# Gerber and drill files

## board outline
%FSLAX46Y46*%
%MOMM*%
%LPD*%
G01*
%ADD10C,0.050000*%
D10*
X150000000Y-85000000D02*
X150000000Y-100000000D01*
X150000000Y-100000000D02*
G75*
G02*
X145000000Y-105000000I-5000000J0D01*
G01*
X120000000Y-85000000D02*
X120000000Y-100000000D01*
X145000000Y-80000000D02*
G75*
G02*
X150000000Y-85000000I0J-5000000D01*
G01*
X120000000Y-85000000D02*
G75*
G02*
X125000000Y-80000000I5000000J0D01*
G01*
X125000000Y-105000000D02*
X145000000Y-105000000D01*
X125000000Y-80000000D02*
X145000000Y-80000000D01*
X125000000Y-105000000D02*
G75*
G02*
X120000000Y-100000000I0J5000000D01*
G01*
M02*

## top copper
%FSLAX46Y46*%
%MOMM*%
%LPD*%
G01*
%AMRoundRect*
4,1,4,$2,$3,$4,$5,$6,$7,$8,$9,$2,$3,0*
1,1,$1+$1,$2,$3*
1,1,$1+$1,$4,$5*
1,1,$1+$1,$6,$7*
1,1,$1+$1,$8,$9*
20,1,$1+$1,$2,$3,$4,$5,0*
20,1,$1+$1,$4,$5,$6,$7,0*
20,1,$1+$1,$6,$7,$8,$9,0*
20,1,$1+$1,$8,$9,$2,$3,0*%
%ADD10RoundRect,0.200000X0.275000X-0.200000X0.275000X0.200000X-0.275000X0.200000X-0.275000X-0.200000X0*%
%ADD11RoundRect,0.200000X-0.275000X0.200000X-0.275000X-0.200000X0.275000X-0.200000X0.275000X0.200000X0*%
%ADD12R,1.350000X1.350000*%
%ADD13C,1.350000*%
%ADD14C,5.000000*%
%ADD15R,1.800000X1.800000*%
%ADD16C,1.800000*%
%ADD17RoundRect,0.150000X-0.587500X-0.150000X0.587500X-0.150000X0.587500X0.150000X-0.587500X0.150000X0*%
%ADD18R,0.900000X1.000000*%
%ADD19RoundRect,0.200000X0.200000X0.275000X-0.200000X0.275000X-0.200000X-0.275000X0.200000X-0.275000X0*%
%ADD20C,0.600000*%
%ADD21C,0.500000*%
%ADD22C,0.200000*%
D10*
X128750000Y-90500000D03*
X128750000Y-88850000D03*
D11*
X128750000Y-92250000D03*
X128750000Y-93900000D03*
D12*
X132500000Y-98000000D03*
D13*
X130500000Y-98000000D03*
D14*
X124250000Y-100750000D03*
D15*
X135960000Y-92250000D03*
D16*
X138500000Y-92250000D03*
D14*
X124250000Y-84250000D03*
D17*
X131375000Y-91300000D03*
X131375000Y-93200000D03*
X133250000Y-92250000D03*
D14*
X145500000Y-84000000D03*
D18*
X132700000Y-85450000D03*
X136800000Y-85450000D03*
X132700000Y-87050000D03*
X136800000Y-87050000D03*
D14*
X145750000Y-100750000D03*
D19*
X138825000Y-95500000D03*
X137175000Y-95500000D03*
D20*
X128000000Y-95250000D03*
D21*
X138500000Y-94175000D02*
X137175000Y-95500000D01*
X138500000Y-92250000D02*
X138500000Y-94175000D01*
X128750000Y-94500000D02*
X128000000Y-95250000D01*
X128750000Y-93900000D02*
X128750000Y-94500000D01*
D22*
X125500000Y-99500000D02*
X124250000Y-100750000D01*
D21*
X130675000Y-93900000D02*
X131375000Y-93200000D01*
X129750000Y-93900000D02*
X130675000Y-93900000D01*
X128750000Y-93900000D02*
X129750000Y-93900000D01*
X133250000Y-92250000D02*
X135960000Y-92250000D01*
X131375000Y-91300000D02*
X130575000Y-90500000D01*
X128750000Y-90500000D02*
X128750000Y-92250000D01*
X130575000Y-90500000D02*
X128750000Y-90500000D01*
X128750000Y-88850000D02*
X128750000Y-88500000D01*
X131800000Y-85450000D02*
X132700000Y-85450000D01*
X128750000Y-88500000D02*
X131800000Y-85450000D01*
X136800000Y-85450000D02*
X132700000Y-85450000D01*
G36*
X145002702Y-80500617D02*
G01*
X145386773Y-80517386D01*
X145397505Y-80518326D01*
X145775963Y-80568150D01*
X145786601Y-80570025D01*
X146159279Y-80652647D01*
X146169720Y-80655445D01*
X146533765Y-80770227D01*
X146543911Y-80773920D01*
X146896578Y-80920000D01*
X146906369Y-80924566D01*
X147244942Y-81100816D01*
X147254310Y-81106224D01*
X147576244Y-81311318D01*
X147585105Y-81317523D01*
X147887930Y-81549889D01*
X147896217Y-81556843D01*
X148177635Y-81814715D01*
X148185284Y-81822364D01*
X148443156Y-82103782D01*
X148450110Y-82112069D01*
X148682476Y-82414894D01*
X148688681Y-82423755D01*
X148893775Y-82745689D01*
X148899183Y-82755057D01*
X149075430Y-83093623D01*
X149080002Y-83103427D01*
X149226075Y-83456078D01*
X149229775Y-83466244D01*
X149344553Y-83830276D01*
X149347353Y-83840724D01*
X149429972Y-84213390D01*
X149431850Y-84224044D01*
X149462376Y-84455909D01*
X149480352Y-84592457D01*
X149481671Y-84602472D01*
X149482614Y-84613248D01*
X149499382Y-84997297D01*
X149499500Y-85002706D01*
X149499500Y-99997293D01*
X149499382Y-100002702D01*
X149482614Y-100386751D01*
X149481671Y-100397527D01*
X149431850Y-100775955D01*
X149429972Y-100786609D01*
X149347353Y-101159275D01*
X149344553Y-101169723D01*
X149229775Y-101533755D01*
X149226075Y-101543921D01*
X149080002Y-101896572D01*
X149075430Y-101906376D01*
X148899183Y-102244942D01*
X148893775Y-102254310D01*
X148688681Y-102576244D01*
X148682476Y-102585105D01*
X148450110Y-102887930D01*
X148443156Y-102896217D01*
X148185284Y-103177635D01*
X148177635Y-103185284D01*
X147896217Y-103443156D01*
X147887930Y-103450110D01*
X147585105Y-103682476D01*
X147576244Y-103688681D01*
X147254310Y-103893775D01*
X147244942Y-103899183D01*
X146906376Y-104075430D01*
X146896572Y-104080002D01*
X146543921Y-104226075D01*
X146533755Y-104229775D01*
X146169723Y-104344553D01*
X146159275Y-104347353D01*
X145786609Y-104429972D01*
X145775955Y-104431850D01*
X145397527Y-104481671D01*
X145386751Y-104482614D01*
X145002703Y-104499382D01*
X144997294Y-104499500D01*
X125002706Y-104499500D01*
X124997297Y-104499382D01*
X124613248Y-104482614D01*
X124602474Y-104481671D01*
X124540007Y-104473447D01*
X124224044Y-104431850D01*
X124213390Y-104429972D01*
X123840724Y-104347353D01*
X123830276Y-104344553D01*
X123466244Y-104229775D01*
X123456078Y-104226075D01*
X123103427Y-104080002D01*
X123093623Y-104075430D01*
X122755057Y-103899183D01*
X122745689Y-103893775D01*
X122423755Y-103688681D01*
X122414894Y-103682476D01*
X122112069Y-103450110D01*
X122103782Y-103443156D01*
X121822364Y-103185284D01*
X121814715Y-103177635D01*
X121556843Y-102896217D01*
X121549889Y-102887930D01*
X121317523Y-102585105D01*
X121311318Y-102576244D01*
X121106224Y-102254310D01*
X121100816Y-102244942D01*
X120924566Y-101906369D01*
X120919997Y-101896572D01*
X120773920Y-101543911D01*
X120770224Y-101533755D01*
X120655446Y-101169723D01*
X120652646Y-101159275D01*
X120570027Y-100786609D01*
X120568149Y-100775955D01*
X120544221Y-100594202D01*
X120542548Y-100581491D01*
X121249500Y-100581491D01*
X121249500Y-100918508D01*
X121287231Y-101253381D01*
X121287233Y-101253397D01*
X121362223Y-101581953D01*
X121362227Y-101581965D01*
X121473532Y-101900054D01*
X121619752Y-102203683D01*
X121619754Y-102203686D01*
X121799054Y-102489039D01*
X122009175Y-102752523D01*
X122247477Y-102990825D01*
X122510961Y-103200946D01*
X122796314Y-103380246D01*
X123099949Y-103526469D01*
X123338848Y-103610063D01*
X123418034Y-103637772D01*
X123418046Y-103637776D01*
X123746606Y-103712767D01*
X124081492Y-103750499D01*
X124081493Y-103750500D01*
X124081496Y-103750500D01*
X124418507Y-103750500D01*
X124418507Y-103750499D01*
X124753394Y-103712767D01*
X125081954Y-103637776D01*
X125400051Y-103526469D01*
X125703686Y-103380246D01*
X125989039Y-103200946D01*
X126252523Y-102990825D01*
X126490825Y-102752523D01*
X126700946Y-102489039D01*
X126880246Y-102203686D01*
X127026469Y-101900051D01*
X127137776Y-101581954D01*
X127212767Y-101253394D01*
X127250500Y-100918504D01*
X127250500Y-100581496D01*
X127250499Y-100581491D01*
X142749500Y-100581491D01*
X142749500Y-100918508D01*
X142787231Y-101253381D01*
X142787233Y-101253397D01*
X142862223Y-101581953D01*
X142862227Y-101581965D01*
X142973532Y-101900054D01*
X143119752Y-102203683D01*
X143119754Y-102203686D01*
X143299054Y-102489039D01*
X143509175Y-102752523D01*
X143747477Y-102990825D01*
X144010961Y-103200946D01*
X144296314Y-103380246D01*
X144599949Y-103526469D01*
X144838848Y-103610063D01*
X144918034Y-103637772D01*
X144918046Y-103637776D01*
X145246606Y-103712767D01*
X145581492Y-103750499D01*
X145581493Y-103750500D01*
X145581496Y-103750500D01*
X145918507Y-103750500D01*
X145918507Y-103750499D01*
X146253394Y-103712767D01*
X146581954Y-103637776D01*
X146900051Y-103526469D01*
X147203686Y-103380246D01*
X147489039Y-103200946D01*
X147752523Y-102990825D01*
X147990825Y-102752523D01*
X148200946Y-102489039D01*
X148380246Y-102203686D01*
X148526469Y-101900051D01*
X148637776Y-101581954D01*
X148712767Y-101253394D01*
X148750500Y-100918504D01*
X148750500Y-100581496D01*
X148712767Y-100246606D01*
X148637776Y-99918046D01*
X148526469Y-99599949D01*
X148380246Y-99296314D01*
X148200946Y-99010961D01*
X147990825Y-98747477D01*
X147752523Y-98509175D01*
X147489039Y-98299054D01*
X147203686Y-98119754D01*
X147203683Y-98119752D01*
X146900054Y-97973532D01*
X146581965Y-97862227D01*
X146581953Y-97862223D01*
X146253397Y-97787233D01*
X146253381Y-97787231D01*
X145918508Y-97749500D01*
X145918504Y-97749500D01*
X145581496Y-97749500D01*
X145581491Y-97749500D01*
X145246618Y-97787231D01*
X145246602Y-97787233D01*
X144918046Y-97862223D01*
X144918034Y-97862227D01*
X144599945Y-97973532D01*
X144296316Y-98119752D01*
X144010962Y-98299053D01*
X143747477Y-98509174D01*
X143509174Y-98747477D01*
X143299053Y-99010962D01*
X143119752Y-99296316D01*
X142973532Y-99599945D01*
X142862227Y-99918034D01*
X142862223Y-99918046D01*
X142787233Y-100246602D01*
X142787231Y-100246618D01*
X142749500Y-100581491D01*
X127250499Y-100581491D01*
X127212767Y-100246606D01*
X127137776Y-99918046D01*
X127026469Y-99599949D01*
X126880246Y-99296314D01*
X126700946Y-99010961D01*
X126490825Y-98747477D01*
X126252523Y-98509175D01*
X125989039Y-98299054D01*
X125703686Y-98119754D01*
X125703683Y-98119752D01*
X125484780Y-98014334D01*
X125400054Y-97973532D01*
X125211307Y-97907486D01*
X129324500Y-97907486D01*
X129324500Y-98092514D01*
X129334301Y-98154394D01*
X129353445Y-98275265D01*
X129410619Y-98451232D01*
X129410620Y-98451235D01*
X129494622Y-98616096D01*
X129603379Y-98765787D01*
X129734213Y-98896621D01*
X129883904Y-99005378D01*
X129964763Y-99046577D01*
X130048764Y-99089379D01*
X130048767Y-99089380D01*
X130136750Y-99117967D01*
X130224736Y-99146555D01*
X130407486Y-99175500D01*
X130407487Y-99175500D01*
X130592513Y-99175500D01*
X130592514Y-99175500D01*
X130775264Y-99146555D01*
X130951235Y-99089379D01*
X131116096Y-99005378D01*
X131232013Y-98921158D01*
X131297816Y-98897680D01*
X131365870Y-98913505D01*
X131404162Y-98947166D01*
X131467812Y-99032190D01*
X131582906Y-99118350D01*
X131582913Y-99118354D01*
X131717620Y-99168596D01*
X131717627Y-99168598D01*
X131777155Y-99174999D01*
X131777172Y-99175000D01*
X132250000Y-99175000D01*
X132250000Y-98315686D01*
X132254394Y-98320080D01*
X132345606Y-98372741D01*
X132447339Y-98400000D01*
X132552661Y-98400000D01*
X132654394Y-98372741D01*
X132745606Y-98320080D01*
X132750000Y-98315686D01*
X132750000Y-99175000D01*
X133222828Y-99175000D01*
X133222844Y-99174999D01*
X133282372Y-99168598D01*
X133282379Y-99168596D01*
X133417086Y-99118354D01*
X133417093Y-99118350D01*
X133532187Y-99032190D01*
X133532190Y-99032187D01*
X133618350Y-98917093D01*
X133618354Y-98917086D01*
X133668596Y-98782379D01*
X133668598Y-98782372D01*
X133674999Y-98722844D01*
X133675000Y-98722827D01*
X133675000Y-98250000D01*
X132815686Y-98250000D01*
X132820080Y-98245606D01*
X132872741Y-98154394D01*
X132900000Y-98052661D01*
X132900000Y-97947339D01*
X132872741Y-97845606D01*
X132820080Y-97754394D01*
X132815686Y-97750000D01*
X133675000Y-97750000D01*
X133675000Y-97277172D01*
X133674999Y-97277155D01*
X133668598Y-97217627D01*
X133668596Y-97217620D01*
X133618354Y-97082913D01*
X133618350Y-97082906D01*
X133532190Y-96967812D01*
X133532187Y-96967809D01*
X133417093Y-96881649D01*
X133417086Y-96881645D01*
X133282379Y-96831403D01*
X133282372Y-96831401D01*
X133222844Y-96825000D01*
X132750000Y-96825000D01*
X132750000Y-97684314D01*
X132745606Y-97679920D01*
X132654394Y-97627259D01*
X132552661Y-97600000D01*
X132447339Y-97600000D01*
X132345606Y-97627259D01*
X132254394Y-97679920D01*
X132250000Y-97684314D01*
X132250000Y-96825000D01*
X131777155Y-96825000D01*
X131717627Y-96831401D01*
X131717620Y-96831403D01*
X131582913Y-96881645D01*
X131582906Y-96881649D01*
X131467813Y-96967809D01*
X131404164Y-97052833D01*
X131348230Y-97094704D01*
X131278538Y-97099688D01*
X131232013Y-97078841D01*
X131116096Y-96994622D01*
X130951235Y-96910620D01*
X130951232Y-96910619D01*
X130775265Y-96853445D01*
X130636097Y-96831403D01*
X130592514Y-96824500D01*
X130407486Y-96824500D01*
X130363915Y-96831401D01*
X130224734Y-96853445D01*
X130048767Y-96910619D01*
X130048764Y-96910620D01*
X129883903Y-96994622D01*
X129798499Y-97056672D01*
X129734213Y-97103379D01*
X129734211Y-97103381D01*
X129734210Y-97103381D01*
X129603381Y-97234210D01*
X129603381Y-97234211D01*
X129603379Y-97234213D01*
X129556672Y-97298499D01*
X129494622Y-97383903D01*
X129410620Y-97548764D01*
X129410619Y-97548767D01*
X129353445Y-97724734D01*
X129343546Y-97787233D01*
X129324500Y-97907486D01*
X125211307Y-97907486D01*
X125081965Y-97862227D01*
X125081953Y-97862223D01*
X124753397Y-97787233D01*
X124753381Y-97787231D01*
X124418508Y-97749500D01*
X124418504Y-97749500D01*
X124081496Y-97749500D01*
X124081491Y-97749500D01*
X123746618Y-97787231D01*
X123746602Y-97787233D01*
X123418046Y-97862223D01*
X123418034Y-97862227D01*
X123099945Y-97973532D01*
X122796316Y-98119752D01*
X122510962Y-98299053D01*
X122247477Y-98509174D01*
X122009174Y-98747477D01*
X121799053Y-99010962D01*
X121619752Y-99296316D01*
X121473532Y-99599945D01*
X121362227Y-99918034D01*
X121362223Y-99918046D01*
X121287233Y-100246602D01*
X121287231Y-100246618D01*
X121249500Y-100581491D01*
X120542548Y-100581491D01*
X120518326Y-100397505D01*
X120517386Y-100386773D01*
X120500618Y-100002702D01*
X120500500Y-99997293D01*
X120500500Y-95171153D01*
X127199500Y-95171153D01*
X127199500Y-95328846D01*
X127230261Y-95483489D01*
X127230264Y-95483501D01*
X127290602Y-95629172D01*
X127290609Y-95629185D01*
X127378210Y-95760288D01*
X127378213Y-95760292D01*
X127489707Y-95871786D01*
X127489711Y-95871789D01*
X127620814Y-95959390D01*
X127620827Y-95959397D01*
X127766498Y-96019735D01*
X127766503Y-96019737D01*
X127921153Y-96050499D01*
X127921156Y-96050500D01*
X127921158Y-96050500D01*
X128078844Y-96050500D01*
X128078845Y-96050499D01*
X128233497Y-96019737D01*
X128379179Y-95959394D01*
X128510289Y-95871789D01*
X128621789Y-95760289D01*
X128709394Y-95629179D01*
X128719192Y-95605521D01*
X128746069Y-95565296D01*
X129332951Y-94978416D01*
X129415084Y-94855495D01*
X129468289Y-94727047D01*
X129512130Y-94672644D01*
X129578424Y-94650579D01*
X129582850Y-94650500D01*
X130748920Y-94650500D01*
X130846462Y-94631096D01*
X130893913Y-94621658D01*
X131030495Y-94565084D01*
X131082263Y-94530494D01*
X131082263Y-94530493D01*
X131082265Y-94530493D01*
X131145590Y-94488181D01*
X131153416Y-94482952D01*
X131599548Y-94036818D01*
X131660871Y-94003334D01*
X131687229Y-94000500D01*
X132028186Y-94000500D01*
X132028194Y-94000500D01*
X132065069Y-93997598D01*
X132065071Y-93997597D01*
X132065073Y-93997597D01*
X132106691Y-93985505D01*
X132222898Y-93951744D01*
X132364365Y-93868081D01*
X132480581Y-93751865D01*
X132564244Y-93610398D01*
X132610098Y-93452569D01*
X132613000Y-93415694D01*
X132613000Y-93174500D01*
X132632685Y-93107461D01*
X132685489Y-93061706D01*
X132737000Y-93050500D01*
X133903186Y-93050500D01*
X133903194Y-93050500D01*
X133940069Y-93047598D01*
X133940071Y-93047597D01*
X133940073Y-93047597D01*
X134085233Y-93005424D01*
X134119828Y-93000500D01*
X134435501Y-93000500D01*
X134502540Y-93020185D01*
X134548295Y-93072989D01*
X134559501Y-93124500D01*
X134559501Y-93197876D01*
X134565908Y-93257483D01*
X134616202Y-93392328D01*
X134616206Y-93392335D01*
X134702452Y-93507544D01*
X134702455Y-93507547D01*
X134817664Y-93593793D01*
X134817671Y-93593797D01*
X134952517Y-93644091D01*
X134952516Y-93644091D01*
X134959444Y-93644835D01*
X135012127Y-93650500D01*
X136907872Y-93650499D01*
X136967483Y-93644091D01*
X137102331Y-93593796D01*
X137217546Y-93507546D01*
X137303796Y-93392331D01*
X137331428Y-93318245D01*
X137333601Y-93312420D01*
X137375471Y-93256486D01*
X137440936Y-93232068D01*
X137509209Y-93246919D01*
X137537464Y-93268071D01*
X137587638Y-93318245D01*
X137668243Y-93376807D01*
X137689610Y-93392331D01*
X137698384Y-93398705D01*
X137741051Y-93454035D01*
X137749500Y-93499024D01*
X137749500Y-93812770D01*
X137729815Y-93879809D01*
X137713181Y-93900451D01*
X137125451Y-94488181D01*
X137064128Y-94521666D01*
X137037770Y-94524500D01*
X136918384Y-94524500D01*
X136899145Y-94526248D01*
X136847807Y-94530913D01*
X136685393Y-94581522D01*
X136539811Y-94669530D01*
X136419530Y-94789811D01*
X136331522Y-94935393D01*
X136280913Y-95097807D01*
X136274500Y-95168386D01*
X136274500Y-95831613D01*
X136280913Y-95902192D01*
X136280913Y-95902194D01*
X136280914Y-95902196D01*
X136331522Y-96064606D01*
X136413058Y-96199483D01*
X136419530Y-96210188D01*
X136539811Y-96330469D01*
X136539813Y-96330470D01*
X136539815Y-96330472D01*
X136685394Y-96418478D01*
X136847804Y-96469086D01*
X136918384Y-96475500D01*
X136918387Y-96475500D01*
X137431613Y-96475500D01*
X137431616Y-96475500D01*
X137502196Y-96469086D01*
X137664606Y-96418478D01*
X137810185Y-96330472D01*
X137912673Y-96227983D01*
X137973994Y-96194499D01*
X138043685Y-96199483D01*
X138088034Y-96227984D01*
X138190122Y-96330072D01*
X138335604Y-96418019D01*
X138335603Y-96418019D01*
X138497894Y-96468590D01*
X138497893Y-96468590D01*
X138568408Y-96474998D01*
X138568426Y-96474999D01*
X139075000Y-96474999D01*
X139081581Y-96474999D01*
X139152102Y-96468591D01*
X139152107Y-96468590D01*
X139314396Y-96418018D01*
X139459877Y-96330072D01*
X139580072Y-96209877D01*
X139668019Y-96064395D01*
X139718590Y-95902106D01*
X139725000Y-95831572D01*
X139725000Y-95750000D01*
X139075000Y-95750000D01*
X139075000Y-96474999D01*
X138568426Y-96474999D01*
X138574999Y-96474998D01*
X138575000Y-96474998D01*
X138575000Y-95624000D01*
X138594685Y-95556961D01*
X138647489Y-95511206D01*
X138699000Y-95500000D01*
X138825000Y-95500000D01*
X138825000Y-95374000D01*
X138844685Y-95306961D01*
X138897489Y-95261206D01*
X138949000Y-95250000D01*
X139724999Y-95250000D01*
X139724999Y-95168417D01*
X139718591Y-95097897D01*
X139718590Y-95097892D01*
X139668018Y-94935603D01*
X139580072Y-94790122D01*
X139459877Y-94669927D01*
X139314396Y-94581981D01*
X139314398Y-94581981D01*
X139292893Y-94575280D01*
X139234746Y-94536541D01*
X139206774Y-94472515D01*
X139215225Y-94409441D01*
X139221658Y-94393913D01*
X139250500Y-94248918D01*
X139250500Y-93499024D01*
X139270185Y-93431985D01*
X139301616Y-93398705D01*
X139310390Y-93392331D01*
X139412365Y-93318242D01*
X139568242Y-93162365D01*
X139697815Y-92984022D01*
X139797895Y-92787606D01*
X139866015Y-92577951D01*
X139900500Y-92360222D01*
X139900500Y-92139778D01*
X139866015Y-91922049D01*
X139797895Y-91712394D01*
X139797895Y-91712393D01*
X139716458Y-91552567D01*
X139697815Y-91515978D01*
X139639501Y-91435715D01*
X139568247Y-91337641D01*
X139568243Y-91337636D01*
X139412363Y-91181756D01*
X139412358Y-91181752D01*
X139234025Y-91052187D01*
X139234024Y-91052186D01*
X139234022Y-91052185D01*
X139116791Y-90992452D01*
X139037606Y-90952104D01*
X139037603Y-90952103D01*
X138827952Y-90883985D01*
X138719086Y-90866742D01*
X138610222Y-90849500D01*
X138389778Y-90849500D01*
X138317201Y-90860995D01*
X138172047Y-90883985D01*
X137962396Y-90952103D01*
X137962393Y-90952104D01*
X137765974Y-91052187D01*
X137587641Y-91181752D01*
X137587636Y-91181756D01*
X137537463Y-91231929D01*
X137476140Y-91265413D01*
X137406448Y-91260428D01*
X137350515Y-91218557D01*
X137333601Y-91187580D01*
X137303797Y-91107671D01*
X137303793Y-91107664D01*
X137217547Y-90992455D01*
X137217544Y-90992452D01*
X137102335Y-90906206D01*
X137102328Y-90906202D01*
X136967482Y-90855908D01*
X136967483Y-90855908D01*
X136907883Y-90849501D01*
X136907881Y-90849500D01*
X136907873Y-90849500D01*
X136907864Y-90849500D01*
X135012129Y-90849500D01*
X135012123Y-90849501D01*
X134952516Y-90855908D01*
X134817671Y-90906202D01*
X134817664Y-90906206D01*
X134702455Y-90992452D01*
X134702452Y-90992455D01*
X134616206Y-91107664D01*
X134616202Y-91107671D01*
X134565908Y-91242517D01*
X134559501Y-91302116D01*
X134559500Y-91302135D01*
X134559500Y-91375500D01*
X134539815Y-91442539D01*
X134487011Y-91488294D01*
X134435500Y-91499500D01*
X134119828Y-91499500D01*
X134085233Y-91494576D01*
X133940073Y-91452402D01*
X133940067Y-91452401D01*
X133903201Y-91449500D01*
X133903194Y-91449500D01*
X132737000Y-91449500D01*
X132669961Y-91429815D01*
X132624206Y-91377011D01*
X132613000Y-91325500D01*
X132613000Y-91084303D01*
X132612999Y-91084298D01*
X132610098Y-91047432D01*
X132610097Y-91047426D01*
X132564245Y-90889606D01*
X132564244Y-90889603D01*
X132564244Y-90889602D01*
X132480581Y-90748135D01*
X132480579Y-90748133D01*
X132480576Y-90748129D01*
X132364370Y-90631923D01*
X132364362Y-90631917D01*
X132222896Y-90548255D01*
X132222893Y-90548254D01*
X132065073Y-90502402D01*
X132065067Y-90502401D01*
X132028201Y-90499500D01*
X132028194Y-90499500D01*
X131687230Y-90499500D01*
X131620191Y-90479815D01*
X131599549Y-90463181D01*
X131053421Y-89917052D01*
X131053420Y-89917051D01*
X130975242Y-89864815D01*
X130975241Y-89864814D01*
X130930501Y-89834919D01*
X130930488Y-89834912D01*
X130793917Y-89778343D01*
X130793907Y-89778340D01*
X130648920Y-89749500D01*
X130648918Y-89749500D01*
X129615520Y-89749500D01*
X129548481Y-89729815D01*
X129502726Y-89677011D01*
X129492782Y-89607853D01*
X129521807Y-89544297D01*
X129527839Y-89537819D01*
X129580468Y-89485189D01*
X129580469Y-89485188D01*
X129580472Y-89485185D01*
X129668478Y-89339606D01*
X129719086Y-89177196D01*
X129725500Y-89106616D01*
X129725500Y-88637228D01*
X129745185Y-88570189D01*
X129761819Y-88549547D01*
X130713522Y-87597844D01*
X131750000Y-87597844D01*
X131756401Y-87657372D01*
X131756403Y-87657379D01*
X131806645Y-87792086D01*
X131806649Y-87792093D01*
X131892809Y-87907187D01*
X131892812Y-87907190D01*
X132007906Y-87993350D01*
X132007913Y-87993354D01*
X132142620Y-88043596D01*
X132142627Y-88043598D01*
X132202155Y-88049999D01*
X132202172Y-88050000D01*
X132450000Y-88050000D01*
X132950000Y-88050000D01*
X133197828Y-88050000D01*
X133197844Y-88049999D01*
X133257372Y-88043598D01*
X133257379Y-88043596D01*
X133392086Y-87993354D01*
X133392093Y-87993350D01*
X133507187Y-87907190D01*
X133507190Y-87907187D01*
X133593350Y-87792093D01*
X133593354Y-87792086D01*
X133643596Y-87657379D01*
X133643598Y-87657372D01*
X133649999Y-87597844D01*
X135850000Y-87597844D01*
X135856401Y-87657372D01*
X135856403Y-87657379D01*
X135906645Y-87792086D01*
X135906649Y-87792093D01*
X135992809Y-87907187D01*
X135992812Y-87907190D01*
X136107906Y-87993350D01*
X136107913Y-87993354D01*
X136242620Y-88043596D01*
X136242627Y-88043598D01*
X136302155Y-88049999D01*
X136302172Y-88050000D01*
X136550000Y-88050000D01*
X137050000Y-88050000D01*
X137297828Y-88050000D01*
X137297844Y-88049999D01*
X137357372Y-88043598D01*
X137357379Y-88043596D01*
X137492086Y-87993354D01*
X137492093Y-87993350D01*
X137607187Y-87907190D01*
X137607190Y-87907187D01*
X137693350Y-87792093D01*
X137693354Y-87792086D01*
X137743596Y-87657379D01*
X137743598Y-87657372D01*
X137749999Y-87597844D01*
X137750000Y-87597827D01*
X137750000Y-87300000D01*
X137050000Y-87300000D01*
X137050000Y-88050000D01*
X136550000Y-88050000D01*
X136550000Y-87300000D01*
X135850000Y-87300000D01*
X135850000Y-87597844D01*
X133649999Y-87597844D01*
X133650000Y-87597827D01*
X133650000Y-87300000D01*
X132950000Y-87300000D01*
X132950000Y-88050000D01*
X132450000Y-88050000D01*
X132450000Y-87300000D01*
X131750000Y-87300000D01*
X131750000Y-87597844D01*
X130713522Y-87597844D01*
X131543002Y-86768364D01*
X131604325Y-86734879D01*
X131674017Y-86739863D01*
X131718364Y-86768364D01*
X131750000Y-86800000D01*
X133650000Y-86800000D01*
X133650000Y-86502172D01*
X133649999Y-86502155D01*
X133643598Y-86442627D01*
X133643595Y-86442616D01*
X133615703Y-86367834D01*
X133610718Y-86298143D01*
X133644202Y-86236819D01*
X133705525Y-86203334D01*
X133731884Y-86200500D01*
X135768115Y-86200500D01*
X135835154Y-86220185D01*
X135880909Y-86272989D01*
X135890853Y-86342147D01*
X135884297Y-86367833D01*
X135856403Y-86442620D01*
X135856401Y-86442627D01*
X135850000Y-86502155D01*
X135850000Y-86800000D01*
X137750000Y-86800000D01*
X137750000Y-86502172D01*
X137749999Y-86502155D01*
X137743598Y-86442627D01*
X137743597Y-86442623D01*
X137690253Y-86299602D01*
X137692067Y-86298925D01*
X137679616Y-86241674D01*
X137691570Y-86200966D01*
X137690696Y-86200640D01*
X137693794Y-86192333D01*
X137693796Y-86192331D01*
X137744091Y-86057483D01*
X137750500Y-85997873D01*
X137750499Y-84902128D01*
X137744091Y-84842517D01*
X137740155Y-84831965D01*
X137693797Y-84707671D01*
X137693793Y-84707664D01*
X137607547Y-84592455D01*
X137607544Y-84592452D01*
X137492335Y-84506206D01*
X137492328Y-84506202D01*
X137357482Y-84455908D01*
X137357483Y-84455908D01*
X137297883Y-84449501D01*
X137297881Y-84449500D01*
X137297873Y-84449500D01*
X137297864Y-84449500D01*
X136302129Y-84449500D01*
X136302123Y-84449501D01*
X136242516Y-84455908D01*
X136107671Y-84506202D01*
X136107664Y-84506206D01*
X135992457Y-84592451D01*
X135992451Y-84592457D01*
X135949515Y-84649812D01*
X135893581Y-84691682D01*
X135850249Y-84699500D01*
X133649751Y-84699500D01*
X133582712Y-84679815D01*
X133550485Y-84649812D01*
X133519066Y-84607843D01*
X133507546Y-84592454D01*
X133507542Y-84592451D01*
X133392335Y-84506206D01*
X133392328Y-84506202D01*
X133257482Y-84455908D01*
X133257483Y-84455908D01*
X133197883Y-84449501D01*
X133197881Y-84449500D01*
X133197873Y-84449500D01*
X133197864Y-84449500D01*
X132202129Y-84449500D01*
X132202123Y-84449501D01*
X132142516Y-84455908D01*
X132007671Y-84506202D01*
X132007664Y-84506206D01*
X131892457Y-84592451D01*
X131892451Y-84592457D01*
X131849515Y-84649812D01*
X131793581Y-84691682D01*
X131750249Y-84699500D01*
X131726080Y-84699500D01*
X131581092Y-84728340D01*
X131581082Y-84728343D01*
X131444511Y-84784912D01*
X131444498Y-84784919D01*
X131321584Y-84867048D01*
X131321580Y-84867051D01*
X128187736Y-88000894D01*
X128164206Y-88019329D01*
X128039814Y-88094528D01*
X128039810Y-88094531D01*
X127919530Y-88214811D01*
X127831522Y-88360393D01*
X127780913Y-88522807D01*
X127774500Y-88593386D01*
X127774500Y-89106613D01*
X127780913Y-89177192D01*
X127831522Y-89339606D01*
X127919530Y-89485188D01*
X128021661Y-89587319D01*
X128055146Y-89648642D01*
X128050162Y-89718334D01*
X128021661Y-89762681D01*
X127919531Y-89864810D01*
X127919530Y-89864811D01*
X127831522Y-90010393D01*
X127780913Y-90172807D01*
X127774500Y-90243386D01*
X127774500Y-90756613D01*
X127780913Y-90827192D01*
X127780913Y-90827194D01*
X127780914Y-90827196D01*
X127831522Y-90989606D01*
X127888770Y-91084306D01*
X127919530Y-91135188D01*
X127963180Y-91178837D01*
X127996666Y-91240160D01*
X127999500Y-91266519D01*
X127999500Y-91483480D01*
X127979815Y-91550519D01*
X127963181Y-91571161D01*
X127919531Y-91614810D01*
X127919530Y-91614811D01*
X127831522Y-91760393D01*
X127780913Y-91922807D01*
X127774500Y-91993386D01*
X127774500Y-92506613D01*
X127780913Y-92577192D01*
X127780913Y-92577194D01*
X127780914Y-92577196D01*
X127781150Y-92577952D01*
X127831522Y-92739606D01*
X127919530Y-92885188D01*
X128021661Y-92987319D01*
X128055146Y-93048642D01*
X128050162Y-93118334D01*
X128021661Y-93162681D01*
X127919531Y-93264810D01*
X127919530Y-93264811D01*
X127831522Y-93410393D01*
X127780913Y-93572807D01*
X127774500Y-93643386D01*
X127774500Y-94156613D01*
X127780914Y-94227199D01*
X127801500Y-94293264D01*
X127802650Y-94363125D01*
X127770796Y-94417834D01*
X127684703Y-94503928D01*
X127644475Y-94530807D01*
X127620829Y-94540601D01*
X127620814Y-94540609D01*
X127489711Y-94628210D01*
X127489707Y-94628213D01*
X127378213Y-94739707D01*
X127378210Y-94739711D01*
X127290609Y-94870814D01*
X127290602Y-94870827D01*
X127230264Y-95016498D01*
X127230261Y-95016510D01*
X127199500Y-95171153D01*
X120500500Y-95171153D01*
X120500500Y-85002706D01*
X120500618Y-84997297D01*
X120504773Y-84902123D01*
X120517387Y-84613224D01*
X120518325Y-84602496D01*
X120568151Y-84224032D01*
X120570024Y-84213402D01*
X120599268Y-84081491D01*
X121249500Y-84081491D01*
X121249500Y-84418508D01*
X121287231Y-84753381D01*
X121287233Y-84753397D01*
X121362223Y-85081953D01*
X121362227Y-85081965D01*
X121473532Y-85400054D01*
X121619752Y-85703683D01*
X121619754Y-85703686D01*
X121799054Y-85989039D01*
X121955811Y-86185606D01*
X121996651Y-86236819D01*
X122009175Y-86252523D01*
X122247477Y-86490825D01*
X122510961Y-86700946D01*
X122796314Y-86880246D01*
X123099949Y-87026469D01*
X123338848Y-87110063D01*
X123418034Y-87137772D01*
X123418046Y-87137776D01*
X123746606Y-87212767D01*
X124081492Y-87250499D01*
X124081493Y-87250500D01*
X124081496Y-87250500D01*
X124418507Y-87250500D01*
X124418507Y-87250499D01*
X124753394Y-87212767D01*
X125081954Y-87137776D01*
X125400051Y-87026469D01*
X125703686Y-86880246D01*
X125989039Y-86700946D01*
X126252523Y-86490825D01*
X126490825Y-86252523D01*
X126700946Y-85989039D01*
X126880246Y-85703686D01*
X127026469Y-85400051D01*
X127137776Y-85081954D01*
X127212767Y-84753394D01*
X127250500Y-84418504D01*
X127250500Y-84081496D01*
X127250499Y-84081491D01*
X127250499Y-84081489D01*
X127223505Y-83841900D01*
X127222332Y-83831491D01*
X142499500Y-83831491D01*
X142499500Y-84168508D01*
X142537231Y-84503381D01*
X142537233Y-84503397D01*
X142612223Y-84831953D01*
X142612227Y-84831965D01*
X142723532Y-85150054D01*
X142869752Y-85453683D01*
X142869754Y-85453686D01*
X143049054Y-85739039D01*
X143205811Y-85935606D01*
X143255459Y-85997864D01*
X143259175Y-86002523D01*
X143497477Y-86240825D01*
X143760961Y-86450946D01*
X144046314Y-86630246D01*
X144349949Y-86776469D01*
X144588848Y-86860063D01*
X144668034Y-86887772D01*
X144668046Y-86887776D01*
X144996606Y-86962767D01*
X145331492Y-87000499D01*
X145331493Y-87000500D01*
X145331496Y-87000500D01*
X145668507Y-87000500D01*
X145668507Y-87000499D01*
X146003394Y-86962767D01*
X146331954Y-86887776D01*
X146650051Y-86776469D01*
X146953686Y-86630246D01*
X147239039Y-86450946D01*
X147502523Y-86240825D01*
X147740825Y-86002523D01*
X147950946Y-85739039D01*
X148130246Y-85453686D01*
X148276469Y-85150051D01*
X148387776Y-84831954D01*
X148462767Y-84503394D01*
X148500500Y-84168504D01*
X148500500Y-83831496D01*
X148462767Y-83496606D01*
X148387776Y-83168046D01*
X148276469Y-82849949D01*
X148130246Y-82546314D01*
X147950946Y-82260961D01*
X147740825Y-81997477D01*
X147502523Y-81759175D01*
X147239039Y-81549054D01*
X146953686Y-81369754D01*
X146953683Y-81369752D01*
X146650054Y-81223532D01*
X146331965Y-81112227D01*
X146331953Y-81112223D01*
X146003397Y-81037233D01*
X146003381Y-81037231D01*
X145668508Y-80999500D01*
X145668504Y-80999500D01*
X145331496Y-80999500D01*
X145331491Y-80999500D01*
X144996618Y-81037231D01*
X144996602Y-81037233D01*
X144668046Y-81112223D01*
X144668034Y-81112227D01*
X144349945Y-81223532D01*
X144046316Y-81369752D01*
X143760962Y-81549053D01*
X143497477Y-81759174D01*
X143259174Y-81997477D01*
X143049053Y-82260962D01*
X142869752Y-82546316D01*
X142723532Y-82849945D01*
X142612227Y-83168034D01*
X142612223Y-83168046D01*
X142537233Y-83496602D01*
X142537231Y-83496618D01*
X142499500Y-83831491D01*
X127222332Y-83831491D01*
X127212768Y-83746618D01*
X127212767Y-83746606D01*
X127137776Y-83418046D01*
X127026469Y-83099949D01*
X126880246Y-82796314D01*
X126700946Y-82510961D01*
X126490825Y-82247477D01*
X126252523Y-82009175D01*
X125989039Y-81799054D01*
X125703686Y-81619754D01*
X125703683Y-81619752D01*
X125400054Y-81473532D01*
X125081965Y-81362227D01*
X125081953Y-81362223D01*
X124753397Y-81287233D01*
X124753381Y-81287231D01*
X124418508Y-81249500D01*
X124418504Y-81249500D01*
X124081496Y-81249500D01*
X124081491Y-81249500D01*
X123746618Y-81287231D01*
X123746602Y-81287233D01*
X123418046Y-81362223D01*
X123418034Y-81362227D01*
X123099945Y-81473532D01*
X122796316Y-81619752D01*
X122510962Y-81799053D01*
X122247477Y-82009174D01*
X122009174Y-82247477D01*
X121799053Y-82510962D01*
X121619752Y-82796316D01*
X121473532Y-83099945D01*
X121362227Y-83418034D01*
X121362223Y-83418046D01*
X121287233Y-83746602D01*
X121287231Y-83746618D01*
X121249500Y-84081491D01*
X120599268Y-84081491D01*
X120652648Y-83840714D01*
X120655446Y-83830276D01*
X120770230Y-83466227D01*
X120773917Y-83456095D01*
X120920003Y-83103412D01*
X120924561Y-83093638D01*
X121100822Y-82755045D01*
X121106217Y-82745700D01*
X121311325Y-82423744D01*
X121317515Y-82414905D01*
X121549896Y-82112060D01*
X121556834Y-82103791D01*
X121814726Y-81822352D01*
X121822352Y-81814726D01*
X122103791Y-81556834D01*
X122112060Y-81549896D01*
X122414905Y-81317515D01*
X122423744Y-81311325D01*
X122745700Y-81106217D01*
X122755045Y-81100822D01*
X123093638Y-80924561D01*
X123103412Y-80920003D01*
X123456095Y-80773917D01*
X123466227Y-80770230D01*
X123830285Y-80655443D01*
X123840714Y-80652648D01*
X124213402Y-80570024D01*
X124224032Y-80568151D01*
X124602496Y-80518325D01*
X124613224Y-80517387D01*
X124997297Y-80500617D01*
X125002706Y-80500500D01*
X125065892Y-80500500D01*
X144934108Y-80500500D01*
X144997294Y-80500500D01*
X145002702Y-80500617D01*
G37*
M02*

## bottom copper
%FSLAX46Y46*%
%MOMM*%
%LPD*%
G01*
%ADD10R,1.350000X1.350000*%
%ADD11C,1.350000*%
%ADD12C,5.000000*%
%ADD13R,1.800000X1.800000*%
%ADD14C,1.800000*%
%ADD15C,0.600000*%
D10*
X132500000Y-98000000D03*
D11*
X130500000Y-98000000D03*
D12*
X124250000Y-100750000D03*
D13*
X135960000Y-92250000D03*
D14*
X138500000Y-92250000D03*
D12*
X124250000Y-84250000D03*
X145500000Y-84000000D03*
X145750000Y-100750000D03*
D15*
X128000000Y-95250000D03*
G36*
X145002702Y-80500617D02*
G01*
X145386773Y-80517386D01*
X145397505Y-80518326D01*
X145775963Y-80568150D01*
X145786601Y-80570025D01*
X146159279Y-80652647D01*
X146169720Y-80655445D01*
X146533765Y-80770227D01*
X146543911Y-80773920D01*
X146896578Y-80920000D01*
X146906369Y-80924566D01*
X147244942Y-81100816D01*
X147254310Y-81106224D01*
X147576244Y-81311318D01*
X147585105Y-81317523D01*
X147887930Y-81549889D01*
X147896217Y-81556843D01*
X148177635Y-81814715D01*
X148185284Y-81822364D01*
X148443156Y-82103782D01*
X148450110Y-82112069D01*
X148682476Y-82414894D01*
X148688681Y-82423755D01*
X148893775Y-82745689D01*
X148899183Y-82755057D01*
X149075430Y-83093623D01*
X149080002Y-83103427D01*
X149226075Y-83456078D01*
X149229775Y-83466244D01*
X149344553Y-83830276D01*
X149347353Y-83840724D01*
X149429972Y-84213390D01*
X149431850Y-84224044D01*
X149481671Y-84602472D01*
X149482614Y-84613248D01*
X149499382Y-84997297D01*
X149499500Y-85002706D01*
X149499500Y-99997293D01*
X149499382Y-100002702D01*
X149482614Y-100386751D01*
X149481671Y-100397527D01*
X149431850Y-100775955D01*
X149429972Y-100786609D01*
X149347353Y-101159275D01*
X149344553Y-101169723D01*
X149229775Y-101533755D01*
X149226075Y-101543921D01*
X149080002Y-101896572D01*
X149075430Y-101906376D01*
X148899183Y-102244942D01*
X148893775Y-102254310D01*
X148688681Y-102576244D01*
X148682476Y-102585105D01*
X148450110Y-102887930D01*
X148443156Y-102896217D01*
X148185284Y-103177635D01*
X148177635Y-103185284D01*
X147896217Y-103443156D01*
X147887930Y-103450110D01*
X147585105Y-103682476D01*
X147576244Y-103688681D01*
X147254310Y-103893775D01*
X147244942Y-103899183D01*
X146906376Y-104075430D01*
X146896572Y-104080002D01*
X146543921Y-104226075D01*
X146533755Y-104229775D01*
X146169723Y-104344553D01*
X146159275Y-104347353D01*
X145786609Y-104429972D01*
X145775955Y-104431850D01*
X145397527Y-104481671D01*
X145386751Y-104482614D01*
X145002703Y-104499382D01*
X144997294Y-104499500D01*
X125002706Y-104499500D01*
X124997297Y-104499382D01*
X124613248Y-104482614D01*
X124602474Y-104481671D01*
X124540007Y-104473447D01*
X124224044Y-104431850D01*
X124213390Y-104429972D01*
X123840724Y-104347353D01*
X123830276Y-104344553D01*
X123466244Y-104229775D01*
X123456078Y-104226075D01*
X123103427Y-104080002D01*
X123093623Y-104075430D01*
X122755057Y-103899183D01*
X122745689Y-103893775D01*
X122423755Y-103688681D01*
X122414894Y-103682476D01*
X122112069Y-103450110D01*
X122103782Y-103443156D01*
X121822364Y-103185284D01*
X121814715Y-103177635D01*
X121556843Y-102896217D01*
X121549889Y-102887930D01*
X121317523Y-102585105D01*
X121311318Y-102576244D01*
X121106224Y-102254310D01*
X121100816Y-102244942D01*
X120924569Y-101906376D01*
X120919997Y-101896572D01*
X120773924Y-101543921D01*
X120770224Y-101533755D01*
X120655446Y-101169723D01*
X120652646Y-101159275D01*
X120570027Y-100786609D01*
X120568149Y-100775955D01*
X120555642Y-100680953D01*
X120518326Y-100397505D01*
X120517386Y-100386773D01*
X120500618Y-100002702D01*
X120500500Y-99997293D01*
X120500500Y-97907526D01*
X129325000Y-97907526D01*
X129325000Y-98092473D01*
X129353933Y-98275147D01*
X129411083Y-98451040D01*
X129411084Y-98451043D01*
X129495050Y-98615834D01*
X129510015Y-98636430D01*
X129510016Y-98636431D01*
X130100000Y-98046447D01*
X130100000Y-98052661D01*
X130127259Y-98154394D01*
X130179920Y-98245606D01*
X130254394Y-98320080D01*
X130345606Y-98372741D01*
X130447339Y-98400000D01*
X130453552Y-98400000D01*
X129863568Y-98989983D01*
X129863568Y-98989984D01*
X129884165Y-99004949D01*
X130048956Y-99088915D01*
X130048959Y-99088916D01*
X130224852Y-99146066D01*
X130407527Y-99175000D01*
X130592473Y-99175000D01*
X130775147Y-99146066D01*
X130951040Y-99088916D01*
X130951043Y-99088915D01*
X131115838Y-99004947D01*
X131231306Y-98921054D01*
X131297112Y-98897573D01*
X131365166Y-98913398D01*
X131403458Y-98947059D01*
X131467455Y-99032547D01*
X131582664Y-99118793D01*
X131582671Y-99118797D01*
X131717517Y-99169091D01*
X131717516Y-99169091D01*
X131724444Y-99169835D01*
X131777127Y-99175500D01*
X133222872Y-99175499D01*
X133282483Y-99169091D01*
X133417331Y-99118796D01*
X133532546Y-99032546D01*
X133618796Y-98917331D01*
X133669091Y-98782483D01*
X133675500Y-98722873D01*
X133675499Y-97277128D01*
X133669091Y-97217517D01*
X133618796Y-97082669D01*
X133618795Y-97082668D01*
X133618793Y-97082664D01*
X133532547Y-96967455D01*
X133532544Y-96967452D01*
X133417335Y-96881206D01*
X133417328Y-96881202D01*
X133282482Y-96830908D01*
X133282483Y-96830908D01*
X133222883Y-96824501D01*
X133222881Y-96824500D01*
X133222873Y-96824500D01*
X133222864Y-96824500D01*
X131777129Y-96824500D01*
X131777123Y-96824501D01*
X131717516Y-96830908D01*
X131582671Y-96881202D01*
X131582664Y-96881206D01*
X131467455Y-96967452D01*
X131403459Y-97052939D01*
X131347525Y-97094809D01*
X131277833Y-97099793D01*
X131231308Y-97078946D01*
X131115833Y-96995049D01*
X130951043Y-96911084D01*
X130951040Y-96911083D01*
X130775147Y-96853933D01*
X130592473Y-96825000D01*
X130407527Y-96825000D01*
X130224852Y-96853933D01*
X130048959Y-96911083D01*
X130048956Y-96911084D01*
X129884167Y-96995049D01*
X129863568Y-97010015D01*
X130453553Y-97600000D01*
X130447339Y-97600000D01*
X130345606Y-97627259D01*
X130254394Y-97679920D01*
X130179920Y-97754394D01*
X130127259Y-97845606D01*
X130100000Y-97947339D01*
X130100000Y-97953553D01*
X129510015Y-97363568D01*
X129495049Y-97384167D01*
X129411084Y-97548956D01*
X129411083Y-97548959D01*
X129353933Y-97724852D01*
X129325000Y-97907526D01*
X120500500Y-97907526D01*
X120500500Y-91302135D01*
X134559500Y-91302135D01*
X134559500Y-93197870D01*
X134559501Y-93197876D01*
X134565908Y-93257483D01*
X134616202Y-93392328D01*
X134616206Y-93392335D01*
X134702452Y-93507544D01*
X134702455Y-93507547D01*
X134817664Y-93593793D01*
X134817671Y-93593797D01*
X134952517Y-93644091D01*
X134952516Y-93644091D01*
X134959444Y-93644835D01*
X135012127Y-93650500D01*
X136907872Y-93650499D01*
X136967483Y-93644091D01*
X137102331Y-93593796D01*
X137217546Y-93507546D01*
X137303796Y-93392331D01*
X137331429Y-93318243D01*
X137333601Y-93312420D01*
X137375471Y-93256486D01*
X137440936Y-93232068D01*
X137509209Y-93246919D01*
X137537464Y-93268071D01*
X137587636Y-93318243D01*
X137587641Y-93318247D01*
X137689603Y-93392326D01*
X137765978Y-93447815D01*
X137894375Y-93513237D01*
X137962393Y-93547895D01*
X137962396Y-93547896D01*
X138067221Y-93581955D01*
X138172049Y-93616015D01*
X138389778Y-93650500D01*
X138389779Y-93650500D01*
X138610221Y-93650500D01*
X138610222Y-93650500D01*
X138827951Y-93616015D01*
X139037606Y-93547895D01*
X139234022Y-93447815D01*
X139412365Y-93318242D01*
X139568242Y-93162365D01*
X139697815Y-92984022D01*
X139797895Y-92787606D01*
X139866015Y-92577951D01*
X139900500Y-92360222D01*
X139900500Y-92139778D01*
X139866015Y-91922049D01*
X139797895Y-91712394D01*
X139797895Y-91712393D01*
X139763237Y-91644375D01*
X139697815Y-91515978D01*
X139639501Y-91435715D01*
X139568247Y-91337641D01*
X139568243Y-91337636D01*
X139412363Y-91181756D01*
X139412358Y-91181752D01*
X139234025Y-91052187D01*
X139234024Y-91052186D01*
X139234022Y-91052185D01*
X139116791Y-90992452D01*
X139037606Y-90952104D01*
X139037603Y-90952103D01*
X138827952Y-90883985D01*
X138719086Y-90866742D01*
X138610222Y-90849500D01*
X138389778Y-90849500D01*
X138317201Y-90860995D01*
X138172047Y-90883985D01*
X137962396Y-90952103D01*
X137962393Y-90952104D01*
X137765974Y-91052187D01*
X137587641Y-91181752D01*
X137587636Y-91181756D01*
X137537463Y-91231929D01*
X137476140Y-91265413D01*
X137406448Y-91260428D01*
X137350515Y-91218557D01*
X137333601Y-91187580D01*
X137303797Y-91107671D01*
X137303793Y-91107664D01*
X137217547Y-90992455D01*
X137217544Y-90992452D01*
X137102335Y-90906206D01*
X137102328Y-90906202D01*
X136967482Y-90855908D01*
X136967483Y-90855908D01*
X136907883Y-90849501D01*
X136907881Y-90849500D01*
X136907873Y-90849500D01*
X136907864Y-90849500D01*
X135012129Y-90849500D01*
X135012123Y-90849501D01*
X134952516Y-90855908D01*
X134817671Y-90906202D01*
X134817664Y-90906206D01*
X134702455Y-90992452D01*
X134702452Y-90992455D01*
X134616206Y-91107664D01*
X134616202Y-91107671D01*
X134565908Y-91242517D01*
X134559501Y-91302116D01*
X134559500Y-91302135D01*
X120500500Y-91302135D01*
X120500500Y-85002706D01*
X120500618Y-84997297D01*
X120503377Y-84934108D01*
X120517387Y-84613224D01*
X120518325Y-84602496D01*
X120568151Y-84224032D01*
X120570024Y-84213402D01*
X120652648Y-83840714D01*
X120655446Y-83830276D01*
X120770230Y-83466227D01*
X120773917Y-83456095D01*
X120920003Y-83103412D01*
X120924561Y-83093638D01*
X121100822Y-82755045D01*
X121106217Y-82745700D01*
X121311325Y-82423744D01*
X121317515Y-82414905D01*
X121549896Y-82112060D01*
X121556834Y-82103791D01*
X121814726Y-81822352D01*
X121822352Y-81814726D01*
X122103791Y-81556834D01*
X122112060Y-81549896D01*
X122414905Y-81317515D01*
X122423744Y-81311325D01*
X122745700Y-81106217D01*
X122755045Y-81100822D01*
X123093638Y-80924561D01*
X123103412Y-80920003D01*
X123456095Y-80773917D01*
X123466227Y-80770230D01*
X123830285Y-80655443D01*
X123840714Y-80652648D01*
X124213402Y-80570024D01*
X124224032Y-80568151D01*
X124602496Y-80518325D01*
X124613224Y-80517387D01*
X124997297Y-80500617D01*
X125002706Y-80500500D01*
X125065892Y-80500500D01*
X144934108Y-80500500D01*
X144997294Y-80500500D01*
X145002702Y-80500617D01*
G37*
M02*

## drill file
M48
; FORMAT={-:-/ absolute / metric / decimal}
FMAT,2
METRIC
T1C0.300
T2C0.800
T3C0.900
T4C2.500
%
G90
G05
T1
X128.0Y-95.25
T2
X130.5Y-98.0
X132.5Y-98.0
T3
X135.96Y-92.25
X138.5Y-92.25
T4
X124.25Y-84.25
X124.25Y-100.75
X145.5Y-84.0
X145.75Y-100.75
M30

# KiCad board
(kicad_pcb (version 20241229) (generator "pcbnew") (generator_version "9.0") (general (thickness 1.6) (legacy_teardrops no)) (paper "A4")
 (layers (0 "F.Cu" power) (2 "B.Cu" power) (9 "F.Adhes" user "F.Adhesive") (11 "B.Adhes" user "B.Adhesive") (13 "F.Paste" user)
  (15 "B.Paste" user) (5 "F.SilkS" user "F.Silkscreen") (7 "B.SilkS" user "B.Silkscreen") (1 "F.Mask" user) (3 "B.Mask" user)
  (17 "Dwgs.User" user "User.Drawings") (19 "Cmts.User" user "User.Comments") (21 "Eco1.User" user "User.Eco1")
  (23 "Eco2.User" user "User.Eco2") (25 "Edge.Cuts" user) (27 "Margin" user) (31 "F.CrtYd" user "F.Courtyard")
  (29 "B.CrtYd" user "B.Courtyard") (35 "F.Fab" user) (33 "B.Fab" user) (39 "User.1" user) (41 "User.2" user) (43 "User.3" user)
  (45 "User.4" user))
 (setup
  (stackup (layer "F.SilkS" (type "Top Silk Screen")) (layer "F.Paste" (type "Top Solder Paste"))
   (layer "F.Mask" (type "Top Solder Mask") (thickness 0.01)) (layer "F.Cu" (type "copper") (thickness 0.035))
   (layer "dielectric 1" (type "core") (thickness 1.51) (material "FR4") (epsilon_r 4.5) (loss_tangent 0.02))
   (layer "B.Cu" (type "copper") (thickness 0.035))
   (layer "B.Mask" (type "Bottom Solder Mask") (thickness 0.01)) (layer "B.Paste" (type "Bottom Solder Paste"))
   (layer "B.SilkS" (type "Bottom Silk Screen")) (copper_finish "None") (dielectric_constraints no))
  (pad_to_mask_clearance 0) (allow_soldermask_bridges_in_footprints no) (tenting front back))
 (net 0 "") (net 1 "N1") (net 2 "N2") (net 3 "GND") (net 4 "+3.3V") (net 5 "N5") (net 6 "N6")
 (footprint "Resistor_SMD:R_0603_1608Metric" (layer "F.Cu") (at 128.75 89.675 90)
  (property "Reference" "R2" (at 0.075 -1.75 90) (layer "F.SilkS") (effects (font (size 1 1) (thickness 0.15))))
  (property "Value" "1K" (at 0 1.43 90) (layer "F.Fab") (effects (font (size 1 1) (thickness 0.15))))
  (pad "1" smd roundrect (at -0.825 0 90) (size 0.8 0.95) (layers "F.Cu" "F.Mask" "F.Paste") (roundrect_rratio 0.25) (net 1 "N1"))
  (pad "2" smd roundrect (at 0.825 0 90) (size 0.8 0.95) (layers "F.Cu" "F.Mask" "F.Paste") (roundrect_rratio 0.25) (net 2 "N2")))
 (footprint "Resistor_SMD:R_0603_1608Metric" (layer "F.Cu") (at 128.75 93.075 -90)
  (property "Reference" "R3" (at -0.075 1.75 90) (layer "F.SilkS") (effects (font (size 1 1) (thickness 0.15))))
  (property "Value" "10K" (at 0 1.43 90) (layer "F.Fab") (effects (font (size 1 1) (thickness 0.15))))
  (pad "1" smd roundrect (at -0.825 0 270) (size 0.8 0.95) (layers "F.Cu" "F.Mask" "F.Paste") (roundrect_rratio 0.25) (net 1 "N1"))
  (pad "2" smd roundrect (at 0.825 0 270) (size 0.8 0.95) (layers "F.Cu" "F.Mask" "F.Paste") (roundrect_rratio 0.25) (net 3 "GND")))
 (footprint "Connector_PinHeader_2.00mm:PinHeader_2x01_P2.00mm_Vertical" (layer "F.Cu") (at 132.5 98 180)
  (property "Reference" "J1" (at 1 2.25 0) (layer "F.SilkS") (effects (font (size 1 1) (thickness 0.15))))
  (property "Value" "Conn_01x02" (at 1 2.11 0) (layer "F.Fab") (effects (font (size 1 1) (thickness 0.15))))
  (pad "1" thru_hole rect (at 0 0 180) (size 1.35 1.35) (drill 0.8) (layers "*.Cu" "*.Mask") (remove_unused_layers no) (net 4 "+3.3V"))
  (pad "2" thru_hole circle (at 2 0 180) (size 1.35 1.35) (drill 0.8) (layers "*.Cu" "*.Mask") (remove_unused_layers no) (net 3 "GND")))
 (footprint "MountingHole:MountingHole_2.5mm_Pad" (layer "F.Cu") (at 124.25 100.75)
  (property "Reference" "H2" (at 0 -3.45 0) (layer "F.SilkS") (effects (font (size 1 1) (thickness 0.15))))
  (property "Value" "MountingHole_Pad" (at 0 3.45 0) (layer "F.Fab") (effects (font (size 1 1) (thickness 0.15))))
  (pad "1" thru_hole circle (at 0 0) (size 5 5) (drill 2.5) (layers "*.Cu" "*.Mask") (remove_unused_layers no) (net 3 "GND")
   (zone_connect 2)))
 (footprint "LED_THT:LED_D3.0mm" (layer "F.Cu") (at 135.96 92.25)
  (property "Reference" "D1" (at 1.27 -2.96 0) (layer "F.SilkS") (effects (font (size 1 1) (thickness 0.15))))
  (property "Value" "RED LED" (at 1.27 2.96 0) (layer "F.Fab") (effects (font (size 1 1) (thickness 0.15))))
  (pad "1" thru_hole rect (at 0 0) (size 1.8 1.8) (drill 0.9) (layers "*.Cu" "*.Mask") (remove_unused_layers no) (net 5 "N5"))
  (pad "2" thru_hole circle (at 2.54 0) (size 1.8 1.8) (drill 0.9) (layers "*.Cu" "*.Mask") (remove_unused_layers no) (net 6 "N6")))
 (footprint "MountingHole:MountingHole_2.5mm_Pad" (layer "F.Cu") (at 124.25 84.25 180)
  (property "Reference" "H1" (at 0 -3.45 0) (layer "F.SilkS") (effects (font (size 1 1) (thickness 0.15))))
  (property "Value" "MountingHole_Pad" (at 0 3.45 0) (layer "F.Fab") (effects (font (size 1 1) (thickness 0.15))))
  (pad "1" thru_hole circle (at 0 0 180) (size 5 5) (drill 2.5) (layers "*.Cu" "*.Mask") (remove_unused_layers no) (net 3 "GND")
   (zone_connect 2)))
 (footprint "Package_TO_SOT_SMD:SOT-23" (layer "F.Cu") (at 132.3125 92.25)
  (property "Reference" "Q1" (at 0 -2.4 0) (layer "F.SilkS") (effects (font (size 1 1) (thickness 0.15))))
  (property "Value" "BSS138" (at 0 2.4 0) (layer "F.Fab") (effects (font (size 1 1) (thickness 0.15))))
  (pad "1" smd roundrect (at -0.9375 -0.95) (size 1.475 0.6) (layers "F.Cu" "F.Mask" "F.Paste") (roundrect_rratio 0.25) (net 1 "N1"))
  (pad "2" smd roundrect (at -0.9375 0.95) (size 1.475 0.6) (layers "F.Cu" "F.Mask" "F.Paste") (roundrect_rratio 0.25) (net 3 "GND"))
  (pad "3" smd roundrect (at 0.9375 0) (size 1.475 0.6) (layers "F.Cu" "F.Mask" "F.Paste") (roundrect_rratio 0.25) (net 5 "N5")))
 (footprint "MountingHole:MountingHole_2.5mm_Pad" (layer "F.Cu") (at 145.5 84 180)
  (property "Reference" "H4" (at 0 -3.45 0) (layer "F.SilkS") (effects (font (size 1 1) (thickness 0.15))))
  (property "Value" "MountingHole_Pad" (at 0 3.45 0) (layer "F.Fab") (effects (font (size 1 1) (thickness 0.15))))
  (pad "1" thru_hole circle (at 0 0 180) (size 5 5) (drill 2.5) (layers "*.Cu" "*.Mask") (remove_unused_layers no) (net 3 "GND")
   (zone_connect 2)))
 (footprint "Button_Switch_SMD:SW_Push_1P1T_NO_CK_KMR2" (layer "F.Cu") (at 134.75 86.25)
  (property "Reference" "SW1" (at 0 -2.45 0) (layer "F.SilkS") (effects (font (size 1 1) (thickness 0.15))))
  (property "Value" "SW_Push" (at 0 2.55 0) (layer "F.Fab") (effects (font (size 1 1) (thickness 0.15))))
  (pad "1" smd rect (at -2.05 -0.8) (size 0.9 1) (layers "F.Cu" "F.Mask" "F.Paste") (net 2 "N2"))
  (pad "1" smd rect (at 2.05 -0.8) (size 0.9 1) (layers "F.Cu" "F.Mask" "F.Paste") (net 2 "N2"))
  (pad "2" smd rect (at -2.05 0.8) (size 0.9 1) (layers "F.Cu" "F.Mask" "F.Paste") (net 4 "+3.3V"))
  (pad "2" smd rect (at 2.05 0.8) (size 0.9 1) (layers "F.Cu" "F.Mask" "F.Paste") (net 4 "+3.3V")))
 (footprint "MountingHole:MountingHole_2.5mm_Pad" (layer "F.Cu") (at 145.75 100.75)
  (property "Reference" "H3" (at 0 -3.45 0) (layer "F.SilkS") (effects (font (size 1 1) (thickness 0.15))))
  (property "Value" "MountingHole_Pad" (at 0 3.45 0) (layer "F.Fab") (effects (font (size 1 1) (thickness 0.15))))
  (pad "1" thru_hole circle (at 0 0) (size 5 5) (drill 2.5) (layers "*.Cu" "*.Mask") (remove_unused_layers no) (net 3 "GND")
   (zone_connect 2)))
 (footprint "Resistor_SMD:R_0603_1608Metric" (layer "F.Cu") (at 138 95.5 180)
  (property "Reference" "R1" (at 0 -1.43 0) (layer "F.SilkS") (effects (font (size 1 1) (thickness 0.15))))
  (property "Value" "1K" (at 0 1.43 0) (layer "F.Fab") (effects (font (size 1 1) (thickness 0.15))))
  (pad "1" smd roundrect (at -0.825 0 180) (size 0.8 0.95) (layers "F.Cu" "F.Mask" "F.Paste") (roundrect_rratio 0.25) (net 4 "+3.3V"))
  (pad "2" smd roundrect (at 0.825 0 180) (size 0.8 0.95) (layers "F.Cu" "F.Mask" "F.Paste") (roundrect_rratio 0.25) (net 6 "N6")))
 (gr_line (start 150 85) (end 150 100) (stroke (width 0.05) (type default)) (layer "Edge.Cuts"))
 (gr_arc (start 150 100) (mid 148.535534 103.535534) (end 145 105) (stroke (width 0.05) (type default)) (layer "Edge.Cuts"))
 (gr_line (start 120 85) (end 120 100) (stroke (width 0.05) (type default)) (layer "Edge.Cuts"))
 (gr_arc (start 145 80) (mid 148.535534 81.464466) (end 150 85) (stroke (width 0.05) (type default)) (layer "Edge.Cuts"))
 (gr_arc (start 120 85) (mid 121.464466 81.464466) (end 125 80) (stroke (width 0.05) (type default)) (layer "Edge.Cuts"))
 (gr_line (start 125 105) (end 145 105) (stroke (width 0.05) (type default)) (layer "Edge.Cuts"))
 (gr_line (start 125 80) (end 145 80) (stroke (width 0.05) (type default)) (layer "Edge.Cuts"))
 (gr_arc (start 125 105) (mid 121.464466 103.535534) (end 120 100) (stroke (width 0.05) (type default)) (layer "Edge.Cuts"))
 (segment (start 138.5 94.175) (end 137.175 95.5) (width 0.5) (layer "F.Cu") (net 6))
 (segment (start 138.5 92.25) (end 138.5 94.175) (width 0.5) (layer "F.Cu") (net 6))
 (segment (start 128.75 94.5) (end 128 95.25) (width 0.5) (layer "F.Cu") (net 3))
 (segment (start 128.75 93.9) (end 128.75 94.5) (width 0.5) (layer "F.Cu") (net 3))
 (segment (start 125.5 99.5) (end 124.25 100.75) (width 0.2) (layer "F.Cu") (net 3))
 (segment (start 130.675 93.9) (end 131.375 93.2) (width 0.5) (layer "F.Cu") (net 3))
 (segment (start 129.75 93.9) (end 130.675 93.9) (width 0.5) (layer "F.Cu") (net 3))
 (segment (start 128.75 93.9) (end 129.75 93.9) (width 0.5) (layer "F.Cu") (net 3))
 (via (at 128 95.25) (size 0.6) (drill 0.3) (layers "F.Cu" "B.Cu") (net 3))
 (segment (start 133.25 92.25) (end 135.96 92.25) (width 0.5) (layer "F.Cu") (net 5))
 (segment (start 131.375 91.3) (end 130.575 90.5) (width 0.5) (layer "F.Cu") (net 1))
 (segment (start 128.75 90.5) (end 128.75 92.25) (width 0.5) (layer "F.Cu") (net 1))
 (segment (start 130.575 90.5) (end 128.75 90.5) (width 0.5) (layer "F.Cu") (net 1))
 (segment (start 128.75 88.85) (end 128.75 88.5) (width 0.5) (layer "F.Cu") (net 2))
 (segment (start 131.8 85.45) (end 132.7 85.45) (width 0.5) (layer "F.Cu") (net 2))
 (segment (start 128.75 88.5) (end 131.8 85.45) (width 0.5) (layer "F.Cu") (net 2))
 (segment (start 136.8 85.45) (end 132.7 85.45) (width 0.5) (layer "F.Cu") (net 2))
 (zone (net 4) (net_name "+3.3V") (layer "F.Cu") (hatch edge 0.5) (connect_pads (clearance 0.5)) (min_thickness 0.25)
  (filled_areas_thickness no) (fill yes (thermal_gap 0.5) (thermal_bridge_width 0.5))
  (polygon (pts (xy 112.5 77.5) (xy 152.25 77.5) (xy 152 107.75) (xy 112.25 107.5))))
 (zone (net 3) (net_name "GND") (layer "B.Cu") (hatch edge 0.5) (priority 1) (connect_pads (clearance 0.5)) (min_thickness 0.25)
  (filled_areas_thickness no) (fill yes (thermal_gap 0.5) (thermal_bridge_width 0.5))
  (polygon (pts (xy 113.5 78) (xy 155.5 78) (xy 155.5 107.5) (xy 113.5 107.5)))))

